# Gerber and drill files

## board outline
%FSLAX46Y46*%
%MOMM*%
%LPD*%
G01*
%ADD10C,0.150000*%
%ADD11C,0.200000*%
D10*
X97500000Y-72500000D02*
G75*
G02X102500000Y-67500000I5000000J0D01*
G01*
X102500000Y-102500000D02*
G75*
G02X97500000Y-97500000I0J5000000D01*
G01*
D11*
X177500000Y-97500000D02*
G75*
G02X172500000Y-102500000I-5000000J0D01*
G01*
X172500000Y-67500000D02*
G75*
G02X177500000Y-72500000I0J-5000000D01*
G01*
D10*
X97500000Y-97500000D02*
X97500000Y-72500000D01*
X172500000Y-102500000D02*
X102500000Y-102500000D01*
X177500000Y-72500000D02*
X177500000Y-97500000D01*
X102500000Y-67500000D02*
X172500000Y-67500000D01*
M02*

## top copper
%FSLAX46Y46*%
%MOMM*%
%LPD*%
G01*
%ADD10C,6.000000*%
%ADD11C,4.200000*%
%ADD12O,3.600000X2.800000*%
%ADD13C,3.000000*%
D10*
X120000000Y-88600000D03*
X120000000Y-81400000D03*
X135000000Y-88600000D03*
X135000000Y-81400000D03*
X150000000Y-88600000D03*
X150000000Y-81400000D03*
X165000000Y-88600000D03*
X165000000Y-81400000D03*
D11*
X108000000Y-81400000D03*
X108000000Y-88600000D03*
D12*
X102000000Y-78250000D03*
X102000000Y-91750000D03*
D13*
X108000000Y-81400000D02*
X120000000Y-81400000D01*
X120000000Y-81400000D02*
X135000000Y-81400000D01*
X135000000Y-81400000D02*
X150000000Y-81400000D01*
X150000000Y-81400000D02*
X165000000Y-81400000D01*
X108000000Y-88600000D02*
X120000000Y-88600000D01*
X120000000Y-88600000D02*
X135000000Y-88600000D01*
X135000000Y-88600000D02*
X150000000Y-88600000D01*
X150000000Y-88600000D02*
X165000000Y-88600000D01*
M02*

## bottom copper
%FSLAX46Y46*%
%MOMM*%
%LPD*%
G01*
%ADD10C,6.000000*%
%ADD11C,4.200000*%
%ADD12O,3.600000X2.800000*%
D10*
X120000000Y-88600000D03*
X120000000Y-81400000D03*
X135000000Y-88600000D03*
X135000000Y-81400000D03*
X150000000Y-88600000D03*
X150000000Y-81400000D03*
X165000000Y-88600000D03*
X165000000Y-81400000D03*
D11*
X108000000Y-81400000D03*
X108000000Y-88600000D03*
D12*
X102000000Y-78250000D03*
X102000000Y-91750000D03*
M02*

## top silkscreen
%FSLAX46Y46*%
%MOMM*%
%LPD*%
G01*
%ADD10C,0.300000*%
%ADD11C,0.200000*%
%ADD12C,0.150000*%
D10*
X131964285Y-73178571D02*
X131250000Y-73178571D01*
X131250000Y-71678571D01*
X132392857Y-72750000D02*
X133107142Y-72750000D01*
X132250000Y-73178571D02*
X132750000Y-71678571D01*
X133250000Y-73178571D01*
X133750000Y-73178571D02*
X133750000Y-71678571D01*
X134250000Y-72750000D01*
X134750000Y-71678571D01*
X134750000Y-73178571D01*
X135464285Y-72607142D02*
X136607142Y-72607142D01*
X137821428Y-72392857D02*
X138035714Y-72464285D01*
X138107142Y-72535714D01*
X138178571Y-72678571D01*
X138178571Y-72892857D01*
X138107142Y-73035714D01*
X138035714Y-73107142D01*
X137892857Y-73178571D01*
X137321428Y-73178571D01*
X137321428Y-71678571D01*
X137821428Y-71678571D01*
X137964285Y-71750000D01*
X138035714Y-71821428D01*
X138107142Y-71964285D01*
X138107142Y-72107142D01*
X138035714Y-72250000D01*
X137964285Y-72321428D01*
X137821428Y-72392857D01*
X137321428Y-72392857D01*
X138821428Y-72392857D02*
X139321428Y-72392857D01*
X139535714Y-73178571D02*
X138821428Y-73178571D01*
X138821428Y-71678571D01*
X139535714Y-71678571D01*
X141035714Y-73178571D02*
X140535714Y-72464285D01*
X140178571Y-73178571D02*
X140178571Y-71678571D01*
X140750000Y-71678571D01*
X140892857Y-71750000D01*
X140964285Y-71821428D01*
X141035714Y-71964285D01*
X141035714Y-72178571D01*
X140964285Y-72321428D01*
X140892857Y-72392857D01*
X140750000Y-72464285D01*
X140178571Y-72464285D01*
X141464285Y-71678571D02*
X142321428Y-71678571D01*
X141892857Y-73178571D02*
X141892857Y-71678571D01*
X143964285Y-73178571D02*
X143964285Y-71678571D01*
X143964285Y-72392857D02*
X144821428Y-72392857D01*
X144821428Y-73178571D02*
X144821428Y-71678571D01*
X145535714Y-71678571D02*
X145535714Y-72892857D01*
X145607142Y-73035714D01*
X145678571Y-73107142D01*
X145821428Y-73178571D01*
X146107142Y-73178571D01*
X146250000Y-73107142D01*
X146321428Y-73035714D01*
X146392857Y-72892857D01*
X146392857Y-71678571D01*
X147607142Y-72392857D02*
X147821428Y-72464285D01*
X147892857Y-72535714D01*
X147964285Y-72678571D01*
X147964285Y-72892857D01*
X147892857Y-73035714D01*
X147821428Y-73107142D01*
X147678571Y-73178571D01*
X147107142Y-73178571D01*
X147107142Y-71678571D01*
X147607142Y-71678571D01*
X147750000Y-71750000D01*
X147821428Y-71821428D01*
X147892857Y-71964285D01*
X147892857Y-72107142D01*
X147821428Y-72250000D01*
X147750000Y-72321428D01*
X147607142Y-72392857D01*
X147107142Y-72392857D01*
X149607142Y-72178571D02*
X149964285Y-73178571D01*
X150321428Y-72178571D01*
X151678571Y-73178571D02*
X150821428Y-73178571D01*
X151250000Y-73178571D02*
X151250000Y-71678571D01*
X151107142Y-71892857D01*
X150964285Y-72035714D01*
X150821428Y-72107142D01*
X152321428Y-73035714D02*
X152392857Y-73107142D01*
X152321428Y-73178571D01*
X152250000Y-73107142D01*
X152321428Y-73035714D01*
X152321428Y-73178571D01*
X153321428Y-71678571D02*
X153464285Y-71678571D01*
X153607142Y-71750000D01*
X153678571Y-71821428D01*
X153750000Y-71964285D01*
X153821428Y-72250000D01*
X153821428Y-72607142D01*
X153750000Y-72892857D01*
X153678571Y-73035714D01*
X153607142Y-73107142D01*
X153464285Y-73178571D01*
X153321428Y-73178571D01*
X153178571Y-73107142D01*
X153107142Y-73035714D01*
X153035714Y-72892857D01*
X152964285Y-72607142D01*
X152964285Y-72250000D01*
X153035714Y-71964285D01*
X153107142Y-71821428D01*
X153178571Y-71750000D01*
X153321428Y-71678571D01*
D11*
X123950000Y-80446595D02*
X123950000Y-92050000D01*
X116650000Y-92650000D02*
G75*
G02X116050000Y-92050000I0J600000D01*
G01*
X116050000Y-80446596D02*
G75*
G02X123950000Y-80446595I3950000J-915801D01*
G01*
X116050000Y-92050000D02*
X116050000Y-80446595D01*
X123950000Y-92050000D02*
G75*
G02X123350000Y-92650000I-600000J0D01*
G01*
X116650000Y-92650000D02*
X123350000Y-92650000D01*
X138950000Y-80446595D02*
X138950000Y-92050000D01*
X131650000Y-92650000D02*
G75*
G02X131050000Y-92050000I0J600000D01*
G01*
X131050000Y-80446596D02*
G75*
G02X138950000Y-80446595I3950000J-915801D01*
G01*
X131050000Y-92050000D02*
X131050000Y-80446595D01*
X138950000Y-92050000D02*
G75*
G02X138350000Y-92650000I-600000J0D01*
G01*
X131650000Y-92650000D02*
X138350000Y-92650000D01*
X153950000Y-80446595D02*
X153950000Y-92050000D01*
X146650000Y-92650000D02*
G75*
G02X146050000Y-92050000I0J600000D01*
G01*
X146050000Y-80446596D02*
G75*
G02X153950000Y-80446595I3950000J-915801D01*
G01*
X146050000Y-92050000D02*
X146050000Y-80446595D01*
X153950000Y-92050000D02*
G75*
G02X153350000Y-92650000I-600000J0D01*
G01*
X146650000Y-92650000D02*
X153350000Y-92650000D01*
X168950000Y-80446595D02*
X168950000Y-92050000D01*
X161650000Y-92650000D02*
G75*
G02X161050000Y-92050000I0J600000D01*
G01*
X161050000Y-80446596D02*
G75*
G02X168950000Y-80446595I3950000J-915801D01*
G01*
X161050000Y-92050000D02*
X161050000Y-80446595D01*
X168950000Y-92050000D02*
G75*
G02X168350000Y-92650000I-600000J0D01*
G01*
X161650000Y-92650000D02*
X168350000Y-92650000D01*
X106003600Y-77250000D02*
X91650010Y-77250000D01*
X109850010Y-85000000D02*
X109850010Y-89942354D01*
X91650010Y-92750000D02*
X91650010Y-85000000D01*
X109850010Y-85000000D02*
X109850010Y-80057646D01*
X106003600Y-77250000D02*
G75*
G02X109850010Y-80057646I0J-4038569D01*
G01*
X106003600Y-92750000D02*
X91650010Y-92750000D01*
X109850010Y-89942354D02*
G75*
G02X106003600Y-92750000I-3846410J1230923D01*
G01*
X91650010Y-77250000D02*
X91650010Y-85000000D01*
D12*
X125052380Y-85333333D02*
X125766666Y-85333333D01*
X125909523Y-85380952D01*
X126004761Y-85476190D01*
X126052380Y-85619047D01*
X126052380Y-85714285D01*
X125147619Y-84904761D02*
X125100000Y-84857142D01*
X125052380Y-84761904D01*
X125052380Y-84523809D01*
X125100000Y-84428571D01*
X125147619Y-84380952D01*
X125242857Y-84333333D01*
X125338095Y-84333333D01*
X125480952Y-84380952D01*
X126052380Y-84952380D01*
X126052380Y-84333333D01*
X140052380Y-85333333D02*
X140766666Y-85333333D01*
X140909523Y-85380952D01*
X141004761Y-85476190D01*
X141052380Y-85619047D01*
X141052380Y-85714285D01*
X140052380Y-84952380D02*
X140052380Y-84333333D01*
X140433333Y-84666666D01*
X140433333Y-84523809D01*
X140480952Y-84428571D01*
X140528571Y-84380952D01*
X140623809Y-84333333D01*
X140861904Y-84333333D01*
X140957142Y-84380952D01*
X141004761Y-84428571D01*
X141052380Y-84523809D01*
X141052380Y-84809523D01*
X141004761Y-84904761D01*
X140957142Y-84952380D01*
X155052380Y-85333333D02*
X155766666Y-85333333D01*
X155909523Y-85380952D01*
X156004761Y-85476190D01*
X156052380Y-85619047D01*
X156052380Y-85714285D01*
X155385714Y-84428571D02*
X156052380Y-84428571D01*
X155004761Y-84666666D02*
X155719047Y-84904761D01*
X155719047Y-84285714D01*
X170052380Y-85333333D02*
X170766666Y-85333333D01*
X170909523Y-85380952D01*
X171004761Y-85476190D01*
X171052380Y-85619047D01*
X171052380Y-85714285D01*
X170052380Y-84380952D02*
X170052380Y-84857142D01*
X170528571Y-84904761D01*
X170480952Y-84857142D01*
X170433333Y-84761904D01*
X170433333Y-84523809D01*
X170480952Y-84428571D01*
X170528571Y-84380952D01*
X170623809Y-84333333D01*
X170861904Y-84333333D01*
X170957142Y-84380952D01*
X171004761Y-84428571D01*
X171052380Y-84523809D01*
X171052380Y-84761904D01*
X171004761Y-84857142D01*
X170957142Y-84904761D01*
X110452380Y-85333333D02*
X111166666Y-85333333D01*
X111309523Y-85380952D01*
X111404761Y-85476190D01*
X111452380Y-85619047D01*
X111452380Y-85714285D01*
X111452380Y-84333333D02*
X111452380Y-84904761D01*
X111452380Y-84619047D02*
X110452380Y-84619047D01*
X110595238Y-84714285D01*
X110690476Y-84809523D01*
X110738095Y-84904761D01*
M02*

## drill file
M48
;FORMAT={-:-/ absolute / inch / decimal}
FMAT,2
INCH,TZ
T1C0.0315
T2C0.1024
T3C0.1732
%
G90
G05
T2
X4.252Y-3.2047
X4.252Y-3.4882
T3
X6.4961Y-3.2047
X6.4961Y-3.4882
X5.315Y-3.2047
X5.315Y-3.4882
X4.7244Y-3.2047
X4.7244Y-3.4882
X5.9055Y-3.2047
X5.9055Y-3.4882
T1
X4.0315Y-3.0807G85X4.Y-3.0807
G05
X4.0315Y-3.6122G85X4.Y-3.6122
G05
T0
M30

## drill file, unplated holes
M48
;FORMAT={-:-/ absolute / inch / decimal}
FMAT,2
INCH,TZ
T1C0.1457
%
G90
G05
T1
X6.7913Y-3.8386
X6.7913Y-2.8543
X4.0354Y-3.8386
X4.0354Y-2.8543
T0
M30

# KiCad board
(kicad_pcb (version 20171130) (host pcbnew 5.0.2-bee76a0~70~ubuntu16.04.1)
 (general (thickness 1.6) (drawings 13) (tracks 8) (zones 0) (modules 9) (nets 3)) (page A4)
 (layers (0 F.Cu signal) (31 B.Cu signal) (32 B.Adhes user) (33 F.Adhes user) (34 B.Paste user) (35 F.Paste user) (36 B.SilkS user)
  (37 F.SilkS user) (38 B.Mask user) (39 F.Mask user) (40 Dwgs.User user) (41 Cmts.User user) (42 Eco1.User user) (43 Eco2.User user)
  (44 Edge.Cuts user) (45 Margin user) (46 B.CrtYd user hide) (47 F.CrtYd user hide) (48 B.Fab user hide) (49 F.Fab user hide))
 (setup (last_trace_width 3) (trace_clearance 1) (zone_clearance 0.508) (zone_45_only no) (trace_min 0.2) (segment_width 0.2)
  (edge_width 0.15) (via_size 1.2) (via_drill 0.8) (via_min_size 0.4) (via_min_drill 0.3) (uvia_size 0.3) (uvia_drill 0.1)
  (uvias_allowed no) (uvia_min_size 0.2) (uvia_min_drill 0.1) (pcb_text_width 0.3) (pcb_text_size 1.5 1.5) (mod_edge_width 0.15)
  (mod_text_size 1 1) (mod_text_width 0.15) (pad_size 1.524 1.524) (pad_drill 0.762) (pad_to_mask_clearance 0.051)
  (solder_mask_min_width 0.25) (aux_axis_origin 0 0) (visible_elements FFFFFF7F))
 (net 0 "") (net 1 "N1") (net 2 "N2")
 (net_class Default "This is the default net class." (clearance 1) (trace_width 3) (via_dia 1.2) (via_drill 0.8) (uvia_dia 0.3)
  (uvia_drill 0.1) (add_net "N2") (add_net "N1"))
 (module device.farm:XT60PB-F (layer F.Cu) (at 120 85 90)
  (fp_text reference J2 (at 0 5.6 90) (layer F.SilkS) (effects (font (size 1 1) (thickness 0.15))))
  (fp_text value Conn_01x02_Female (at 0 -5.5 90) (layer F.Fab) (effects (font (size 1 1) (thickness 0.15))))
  (fp_line (start 4.553405 3.95) (end -7.05 3.95) (layer F.SilkS) (width 0.2))
  (fp_arc (start -7.05 -3.35) (end -7.05 -3.95) (angle -90.00000008) (layer F.SilkS) (width 0.2))
  (fp_arc (start 3.637603 0) (end 4.553405 3.95) (angle -153.8933811) (layer F.SilkS) (width 0.2))
  (fp_line (start -7.05 -3.95) (end 4.553405 -3.95) (layer F.SilkS) (width 0.2))
  (fp_arc (start -7.05 3.35) (end -7.65 3.35) (angle -90) (layer F.SilkS) (width 0.2))
  (fp_line (start -7.65 -3.35) (end -7.65 3.35) (layer F.SilkS) (width 0.2))
  (pad 2 thru_hole circle (at -3.6 0 90) (size 6 6) (drill 4.4) (layers *.Cu *.Mask) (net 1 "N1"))
  (pad 1 thru_hole circle (at 3.6 0 90) (size 6 6) (drill 4.4) (layers *.Cu *.Mask) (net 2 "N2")))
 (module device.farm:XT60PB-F (layer F.Cu) (at 135 85 90)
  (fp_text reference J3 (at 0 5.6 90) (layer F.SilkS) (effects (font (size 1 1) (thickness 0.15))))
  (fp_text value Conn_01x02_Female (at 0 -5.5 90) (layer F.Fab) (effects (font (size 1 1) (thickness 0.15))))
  (fp_line (start 4.553405 3.95) (end -7.05 3.95) (layer F.SilkS) (width 0.2))
  (fp_arc (start -7.05 -3.35) (end -7.05 -3.95) (angle -90.00000008) (layer F.SilkS) (width 0.2))
  (fp_arc (start 3.637603 0) (end 4.553405 3.95) (angle -153.8933811) (layer F.SilkS) (width 0.2))
  (fp_line (start -7.05 -3.95) (end 4.553405 -3.95) (layer F.SilkS) (width 0.2))
  (fp_arc (start -7.05 3.35) (end -7.65 3.35) (angle -90) (layer F.SilkS) (width 0.2))
  (fp_line (start -7.65 -3.35) (end -7.65 3.35) (layer F.SilkS) (width 0.2))
  (pad 2 thru_hole circle (at -3.6 0 90) (size 6 6) (drill 4.4) (layers *.Cu *.Mask) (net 1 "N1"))
  (pad 1 thru_hole circle (at 3.6 0 90) (size 6 6) (drill 4.4) (layers *.Cu *.Mask) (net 2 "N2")))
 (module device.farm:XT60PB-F (layer F.Cu) (at 150 85 90)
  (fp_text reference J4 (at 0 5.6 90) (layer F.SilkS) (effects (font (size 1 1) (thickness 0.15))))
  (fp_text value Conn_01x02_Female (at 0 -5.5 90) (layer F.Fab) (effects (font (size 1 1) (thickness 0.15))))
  (fp_line (start 4.553405 3.95) (end -7.05 3.95) (layer F.SilkS) (width 0.2))
  (fp_arc (start -7.05 -3.35) (end -7.05 -3.95) (angle -90.00000008) (layer F.SilkS) (width 0.2))
  (fp_arc (start 3.637603 0) (end 4.553405 3.95) (angle -153.8933811) (layer F.SilkS) (width 0.2))
  (fp_line (start -7.05 -3.95) (end 4.553405 -3.95) (layer F.SilkS) (width 0.2))
  (fp_arc (start -7.05 3.35) (end -7.65 3.35) (angle -90) (layer F.SilkS) (width 0.2))
  (fp_line (start -7.65 -3.35) (end -7.65 3.35) (layer F.SilkS) (width 0.2))
  (pad 2 thru_hole circle (at -3.6 0 90) (size 6 6) (drill 4.4) (layers *.Cu *.Mask) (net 1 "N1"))
  (pad 1 thru_hole circle (at 3.6 0 90) (size 6 6) (drill 4.4) (layers *.Cu *.Mask) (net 2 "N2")))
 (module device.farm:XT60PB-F (layer F.Cu) (at 165 85 90)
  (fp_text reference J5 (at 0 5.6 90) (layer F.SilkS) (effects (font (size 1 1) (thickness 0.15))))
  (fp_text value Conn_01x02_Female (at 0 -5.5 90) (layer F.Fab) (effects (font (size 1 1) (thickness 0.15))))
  (fp_line (start 4.553405 3.95) (end -7.05 3.95) (layer F.SilkS) (width 0.2))
  (fp_arc (start -7.05 -3.35) (end -7.05 -3.95) (angle -90.00000008) (layer F.SilkS) (width 0.2))
  (fp_arc (start 3.637603 0) (end 4.553405 3.95) (angle -153.8933811) (layer F.SilkS) (width 0.2))
  (fp_line (start -7.05 -3.95) (end 4.553405 -3.95) (layer F.SilkS) (width 0.2))
  (fp_arc (start -7.05 3.35) (end -7.65 3.35) (angle -90) (layer F.SilkS) (width 0.2))
  (fp_line (start -7.65 -3.35) (end -7.65 3.35) (layer F.SilkS) (width 0.2))
  (pad 2 thru_hole circle (at -3.6 0 90) (size 6 6) (drill 4.4) (layers *.Cu *.Mask) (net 1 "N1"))
  (pad 1 thru_hole circle (at 3.6 0 90) (size 6 6) (drill 4.4) (layers *.Cu *.Mask) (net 2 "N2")))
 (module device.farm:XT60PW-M (layer F.Cu) (at 108 85 270)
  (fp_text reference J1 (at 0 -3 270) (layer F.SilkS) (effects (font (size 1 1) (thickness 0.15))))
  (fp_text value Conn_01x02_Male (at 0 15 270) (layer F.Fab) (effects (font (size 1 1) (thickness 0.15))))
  (fp_line (start -7.75 1.9964) (end -7.75 16.34999) (layer F.SilkS) (width 0.2))
  (fp_line (start 0 -1.85001) (end 4.942354 -1.85001) (layer F.SilkS) (width 0.2))
  (fp_line (start 7.75 16.34999) (end 0 16.34999) (layer F.SilkS) (width 0.2))
  (fp_line (start 0 -1.85001) (end -4.942354 -1.85001) (layer F.SilkS) (width 0.2))
  (fp_arc (start -3.711431 1.9964) (end -4.942354 -1.85001) (angle -72.25435427) (layer F.SilkS) (width 0.2))
  (fp_line (start 7.75 1.9964) (end 7.75 16.34999) (layer F.SilkS) (width 0.2))
  (fp_arc (start 3.711431 1.9964) (end 7.75 1.9964) (angle -72.25435427) (layer F.SilkS) (width 0.2))
  (fp_line (start -7.75 16.34999) (end 0 16.34999) (layer F.SilkS) (width 0.2))
  (pad 1 thru_hole circle (at -3.6 0 270) (size 4.2 4.2) (drill 2.6) (layers *.Cu *.Mask) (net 2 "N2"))
  (pad 2 thru_hole circle (at 3.6 0 270) (size 4.2 4.2) (drill 2.6) (layers *.Cu *.Mask) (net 1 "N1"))
  (pad "" thru_hole oval (at -6.75 6 270) (size 2.8 3.6) (drill oval 0.8 1.6) (layers *.Cu *.Mask))
  (pad "" thru_hole oval (at 6.75 6 270) (size 2.8 3.6) (drill oval 0.8 1.6) (layers *.Cu *.Mask)))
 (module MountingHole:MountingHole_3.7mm (layer F.Cu) (at 102.5 72.5)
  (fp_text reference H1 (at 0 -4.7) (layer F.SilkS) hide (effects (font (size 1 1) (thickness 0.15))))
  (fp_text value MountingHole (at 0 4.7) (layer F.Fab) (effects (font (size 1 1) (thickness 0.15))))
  (pad 1 np_thru_hole circle (at 0 0) (size 3.7 3.7) (drill 3.7) (layers *.Cu *.Mask)))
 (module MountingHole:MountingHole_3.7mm (layer F.Cu) (at 102.5 97.5)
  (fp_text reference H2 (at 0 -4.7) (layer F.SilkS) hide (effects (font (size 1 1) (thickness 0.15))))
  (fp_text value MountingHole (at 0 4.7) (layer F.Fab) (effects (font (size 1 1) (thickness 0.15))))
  (pad 1 np_thru_hole circle (at 0 0) (size 3.7 3.7) (drill 3.7) (layers *.Cu *.Mask)))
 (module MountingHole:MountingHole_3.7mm (layer F.Cu) (at 172.5 72.5)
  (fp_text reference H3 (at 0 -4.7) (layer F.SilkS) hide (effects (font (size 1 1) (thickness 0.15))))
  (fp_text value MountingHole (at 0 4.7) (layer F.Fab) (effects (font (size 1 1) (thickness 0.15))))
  (pad 1 np_thru_hole circle (at 0 0) (size 3.7 3.7) (drill 3.7) (layers *.Cu *.Mask)))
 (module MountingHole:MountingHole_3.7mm (layer F.Cu) (at 172.5 97.5)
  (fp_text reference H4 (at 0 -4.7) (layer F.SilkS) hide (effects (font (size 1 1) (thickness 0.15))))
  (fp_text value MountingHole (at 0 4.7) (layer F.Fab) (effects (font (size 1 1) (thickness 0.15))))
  (pad 1 np_thru_hole circle (at 0 0) (size 3.7 3.7) (drill 3.7) (layers *.Cu *.Mask)))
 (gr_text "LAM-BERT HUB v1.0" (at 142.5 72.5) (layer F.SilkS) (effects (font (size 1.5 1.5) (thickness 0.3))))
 (gr_arc (start 102.5 72.5) (end 102.5 67.5) (angle -90) (layer Edge.Cuts) (width 0.15))
 (gr_arc (start 102.5 97.5) (end 97.5 97.5) (angle -90) (layer Edge.Cuts) (width 0.15))
 (gr_arc (start 172.5 97.5) (end 172.5 102.5) (angle -90) (layer Edge.Cuts) (width 0.2))
 (gr_arc (start 172.5 72.5) (end 177.5 72.5) (angle -90) (layer Edge.Cuts) (width 0.2))
 (gr_line (start 97.5 97.5) (end 97.5 72.5) (layer Edge.Cuts) (width 0.15))
 (gr_line (start 172.5 102.5) (end 102.5 102.5) (layer Edge.Cuts) (width 0.15))
 (gr_line (start 177.5 72.5) (end 177.5 97.5) (layer Edge.Cuts) (width 0.15))
 (gr_line (start 102.5 67.5) (end 172.5 67.5) (layer Edge.Cuts) (width 0.15))
 (segment (start 108 81.4) (end 120 81.4) (width 3) (layer F.Cu) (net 2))
 (segment (start 120 81.4) (end 135 81.4) (width 3) (layer F.Cu) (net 2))
 (segment (start 135 81.4) (end 150 81.4) (width 3) (layer F.Cu) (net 2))
 (segment (start 150 81.4) (end 165 81.4) (width 3) (layer F.Cu) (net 2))
 (segment (start 108 88.6) (end 120 88.6) (width 3) (layer F.Cu) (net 1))
 (segment (start 120 88.6) (end 135 88.6) (width 3) (layer F.Cu) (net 1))
 (segment (start 135 88.6) (end 150 88.6) (width 3) (layer F.Cu) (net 1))
 (segment (start 150 88.6) (end 165 88.6) (width 3) (layer F.Cu) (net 1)))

